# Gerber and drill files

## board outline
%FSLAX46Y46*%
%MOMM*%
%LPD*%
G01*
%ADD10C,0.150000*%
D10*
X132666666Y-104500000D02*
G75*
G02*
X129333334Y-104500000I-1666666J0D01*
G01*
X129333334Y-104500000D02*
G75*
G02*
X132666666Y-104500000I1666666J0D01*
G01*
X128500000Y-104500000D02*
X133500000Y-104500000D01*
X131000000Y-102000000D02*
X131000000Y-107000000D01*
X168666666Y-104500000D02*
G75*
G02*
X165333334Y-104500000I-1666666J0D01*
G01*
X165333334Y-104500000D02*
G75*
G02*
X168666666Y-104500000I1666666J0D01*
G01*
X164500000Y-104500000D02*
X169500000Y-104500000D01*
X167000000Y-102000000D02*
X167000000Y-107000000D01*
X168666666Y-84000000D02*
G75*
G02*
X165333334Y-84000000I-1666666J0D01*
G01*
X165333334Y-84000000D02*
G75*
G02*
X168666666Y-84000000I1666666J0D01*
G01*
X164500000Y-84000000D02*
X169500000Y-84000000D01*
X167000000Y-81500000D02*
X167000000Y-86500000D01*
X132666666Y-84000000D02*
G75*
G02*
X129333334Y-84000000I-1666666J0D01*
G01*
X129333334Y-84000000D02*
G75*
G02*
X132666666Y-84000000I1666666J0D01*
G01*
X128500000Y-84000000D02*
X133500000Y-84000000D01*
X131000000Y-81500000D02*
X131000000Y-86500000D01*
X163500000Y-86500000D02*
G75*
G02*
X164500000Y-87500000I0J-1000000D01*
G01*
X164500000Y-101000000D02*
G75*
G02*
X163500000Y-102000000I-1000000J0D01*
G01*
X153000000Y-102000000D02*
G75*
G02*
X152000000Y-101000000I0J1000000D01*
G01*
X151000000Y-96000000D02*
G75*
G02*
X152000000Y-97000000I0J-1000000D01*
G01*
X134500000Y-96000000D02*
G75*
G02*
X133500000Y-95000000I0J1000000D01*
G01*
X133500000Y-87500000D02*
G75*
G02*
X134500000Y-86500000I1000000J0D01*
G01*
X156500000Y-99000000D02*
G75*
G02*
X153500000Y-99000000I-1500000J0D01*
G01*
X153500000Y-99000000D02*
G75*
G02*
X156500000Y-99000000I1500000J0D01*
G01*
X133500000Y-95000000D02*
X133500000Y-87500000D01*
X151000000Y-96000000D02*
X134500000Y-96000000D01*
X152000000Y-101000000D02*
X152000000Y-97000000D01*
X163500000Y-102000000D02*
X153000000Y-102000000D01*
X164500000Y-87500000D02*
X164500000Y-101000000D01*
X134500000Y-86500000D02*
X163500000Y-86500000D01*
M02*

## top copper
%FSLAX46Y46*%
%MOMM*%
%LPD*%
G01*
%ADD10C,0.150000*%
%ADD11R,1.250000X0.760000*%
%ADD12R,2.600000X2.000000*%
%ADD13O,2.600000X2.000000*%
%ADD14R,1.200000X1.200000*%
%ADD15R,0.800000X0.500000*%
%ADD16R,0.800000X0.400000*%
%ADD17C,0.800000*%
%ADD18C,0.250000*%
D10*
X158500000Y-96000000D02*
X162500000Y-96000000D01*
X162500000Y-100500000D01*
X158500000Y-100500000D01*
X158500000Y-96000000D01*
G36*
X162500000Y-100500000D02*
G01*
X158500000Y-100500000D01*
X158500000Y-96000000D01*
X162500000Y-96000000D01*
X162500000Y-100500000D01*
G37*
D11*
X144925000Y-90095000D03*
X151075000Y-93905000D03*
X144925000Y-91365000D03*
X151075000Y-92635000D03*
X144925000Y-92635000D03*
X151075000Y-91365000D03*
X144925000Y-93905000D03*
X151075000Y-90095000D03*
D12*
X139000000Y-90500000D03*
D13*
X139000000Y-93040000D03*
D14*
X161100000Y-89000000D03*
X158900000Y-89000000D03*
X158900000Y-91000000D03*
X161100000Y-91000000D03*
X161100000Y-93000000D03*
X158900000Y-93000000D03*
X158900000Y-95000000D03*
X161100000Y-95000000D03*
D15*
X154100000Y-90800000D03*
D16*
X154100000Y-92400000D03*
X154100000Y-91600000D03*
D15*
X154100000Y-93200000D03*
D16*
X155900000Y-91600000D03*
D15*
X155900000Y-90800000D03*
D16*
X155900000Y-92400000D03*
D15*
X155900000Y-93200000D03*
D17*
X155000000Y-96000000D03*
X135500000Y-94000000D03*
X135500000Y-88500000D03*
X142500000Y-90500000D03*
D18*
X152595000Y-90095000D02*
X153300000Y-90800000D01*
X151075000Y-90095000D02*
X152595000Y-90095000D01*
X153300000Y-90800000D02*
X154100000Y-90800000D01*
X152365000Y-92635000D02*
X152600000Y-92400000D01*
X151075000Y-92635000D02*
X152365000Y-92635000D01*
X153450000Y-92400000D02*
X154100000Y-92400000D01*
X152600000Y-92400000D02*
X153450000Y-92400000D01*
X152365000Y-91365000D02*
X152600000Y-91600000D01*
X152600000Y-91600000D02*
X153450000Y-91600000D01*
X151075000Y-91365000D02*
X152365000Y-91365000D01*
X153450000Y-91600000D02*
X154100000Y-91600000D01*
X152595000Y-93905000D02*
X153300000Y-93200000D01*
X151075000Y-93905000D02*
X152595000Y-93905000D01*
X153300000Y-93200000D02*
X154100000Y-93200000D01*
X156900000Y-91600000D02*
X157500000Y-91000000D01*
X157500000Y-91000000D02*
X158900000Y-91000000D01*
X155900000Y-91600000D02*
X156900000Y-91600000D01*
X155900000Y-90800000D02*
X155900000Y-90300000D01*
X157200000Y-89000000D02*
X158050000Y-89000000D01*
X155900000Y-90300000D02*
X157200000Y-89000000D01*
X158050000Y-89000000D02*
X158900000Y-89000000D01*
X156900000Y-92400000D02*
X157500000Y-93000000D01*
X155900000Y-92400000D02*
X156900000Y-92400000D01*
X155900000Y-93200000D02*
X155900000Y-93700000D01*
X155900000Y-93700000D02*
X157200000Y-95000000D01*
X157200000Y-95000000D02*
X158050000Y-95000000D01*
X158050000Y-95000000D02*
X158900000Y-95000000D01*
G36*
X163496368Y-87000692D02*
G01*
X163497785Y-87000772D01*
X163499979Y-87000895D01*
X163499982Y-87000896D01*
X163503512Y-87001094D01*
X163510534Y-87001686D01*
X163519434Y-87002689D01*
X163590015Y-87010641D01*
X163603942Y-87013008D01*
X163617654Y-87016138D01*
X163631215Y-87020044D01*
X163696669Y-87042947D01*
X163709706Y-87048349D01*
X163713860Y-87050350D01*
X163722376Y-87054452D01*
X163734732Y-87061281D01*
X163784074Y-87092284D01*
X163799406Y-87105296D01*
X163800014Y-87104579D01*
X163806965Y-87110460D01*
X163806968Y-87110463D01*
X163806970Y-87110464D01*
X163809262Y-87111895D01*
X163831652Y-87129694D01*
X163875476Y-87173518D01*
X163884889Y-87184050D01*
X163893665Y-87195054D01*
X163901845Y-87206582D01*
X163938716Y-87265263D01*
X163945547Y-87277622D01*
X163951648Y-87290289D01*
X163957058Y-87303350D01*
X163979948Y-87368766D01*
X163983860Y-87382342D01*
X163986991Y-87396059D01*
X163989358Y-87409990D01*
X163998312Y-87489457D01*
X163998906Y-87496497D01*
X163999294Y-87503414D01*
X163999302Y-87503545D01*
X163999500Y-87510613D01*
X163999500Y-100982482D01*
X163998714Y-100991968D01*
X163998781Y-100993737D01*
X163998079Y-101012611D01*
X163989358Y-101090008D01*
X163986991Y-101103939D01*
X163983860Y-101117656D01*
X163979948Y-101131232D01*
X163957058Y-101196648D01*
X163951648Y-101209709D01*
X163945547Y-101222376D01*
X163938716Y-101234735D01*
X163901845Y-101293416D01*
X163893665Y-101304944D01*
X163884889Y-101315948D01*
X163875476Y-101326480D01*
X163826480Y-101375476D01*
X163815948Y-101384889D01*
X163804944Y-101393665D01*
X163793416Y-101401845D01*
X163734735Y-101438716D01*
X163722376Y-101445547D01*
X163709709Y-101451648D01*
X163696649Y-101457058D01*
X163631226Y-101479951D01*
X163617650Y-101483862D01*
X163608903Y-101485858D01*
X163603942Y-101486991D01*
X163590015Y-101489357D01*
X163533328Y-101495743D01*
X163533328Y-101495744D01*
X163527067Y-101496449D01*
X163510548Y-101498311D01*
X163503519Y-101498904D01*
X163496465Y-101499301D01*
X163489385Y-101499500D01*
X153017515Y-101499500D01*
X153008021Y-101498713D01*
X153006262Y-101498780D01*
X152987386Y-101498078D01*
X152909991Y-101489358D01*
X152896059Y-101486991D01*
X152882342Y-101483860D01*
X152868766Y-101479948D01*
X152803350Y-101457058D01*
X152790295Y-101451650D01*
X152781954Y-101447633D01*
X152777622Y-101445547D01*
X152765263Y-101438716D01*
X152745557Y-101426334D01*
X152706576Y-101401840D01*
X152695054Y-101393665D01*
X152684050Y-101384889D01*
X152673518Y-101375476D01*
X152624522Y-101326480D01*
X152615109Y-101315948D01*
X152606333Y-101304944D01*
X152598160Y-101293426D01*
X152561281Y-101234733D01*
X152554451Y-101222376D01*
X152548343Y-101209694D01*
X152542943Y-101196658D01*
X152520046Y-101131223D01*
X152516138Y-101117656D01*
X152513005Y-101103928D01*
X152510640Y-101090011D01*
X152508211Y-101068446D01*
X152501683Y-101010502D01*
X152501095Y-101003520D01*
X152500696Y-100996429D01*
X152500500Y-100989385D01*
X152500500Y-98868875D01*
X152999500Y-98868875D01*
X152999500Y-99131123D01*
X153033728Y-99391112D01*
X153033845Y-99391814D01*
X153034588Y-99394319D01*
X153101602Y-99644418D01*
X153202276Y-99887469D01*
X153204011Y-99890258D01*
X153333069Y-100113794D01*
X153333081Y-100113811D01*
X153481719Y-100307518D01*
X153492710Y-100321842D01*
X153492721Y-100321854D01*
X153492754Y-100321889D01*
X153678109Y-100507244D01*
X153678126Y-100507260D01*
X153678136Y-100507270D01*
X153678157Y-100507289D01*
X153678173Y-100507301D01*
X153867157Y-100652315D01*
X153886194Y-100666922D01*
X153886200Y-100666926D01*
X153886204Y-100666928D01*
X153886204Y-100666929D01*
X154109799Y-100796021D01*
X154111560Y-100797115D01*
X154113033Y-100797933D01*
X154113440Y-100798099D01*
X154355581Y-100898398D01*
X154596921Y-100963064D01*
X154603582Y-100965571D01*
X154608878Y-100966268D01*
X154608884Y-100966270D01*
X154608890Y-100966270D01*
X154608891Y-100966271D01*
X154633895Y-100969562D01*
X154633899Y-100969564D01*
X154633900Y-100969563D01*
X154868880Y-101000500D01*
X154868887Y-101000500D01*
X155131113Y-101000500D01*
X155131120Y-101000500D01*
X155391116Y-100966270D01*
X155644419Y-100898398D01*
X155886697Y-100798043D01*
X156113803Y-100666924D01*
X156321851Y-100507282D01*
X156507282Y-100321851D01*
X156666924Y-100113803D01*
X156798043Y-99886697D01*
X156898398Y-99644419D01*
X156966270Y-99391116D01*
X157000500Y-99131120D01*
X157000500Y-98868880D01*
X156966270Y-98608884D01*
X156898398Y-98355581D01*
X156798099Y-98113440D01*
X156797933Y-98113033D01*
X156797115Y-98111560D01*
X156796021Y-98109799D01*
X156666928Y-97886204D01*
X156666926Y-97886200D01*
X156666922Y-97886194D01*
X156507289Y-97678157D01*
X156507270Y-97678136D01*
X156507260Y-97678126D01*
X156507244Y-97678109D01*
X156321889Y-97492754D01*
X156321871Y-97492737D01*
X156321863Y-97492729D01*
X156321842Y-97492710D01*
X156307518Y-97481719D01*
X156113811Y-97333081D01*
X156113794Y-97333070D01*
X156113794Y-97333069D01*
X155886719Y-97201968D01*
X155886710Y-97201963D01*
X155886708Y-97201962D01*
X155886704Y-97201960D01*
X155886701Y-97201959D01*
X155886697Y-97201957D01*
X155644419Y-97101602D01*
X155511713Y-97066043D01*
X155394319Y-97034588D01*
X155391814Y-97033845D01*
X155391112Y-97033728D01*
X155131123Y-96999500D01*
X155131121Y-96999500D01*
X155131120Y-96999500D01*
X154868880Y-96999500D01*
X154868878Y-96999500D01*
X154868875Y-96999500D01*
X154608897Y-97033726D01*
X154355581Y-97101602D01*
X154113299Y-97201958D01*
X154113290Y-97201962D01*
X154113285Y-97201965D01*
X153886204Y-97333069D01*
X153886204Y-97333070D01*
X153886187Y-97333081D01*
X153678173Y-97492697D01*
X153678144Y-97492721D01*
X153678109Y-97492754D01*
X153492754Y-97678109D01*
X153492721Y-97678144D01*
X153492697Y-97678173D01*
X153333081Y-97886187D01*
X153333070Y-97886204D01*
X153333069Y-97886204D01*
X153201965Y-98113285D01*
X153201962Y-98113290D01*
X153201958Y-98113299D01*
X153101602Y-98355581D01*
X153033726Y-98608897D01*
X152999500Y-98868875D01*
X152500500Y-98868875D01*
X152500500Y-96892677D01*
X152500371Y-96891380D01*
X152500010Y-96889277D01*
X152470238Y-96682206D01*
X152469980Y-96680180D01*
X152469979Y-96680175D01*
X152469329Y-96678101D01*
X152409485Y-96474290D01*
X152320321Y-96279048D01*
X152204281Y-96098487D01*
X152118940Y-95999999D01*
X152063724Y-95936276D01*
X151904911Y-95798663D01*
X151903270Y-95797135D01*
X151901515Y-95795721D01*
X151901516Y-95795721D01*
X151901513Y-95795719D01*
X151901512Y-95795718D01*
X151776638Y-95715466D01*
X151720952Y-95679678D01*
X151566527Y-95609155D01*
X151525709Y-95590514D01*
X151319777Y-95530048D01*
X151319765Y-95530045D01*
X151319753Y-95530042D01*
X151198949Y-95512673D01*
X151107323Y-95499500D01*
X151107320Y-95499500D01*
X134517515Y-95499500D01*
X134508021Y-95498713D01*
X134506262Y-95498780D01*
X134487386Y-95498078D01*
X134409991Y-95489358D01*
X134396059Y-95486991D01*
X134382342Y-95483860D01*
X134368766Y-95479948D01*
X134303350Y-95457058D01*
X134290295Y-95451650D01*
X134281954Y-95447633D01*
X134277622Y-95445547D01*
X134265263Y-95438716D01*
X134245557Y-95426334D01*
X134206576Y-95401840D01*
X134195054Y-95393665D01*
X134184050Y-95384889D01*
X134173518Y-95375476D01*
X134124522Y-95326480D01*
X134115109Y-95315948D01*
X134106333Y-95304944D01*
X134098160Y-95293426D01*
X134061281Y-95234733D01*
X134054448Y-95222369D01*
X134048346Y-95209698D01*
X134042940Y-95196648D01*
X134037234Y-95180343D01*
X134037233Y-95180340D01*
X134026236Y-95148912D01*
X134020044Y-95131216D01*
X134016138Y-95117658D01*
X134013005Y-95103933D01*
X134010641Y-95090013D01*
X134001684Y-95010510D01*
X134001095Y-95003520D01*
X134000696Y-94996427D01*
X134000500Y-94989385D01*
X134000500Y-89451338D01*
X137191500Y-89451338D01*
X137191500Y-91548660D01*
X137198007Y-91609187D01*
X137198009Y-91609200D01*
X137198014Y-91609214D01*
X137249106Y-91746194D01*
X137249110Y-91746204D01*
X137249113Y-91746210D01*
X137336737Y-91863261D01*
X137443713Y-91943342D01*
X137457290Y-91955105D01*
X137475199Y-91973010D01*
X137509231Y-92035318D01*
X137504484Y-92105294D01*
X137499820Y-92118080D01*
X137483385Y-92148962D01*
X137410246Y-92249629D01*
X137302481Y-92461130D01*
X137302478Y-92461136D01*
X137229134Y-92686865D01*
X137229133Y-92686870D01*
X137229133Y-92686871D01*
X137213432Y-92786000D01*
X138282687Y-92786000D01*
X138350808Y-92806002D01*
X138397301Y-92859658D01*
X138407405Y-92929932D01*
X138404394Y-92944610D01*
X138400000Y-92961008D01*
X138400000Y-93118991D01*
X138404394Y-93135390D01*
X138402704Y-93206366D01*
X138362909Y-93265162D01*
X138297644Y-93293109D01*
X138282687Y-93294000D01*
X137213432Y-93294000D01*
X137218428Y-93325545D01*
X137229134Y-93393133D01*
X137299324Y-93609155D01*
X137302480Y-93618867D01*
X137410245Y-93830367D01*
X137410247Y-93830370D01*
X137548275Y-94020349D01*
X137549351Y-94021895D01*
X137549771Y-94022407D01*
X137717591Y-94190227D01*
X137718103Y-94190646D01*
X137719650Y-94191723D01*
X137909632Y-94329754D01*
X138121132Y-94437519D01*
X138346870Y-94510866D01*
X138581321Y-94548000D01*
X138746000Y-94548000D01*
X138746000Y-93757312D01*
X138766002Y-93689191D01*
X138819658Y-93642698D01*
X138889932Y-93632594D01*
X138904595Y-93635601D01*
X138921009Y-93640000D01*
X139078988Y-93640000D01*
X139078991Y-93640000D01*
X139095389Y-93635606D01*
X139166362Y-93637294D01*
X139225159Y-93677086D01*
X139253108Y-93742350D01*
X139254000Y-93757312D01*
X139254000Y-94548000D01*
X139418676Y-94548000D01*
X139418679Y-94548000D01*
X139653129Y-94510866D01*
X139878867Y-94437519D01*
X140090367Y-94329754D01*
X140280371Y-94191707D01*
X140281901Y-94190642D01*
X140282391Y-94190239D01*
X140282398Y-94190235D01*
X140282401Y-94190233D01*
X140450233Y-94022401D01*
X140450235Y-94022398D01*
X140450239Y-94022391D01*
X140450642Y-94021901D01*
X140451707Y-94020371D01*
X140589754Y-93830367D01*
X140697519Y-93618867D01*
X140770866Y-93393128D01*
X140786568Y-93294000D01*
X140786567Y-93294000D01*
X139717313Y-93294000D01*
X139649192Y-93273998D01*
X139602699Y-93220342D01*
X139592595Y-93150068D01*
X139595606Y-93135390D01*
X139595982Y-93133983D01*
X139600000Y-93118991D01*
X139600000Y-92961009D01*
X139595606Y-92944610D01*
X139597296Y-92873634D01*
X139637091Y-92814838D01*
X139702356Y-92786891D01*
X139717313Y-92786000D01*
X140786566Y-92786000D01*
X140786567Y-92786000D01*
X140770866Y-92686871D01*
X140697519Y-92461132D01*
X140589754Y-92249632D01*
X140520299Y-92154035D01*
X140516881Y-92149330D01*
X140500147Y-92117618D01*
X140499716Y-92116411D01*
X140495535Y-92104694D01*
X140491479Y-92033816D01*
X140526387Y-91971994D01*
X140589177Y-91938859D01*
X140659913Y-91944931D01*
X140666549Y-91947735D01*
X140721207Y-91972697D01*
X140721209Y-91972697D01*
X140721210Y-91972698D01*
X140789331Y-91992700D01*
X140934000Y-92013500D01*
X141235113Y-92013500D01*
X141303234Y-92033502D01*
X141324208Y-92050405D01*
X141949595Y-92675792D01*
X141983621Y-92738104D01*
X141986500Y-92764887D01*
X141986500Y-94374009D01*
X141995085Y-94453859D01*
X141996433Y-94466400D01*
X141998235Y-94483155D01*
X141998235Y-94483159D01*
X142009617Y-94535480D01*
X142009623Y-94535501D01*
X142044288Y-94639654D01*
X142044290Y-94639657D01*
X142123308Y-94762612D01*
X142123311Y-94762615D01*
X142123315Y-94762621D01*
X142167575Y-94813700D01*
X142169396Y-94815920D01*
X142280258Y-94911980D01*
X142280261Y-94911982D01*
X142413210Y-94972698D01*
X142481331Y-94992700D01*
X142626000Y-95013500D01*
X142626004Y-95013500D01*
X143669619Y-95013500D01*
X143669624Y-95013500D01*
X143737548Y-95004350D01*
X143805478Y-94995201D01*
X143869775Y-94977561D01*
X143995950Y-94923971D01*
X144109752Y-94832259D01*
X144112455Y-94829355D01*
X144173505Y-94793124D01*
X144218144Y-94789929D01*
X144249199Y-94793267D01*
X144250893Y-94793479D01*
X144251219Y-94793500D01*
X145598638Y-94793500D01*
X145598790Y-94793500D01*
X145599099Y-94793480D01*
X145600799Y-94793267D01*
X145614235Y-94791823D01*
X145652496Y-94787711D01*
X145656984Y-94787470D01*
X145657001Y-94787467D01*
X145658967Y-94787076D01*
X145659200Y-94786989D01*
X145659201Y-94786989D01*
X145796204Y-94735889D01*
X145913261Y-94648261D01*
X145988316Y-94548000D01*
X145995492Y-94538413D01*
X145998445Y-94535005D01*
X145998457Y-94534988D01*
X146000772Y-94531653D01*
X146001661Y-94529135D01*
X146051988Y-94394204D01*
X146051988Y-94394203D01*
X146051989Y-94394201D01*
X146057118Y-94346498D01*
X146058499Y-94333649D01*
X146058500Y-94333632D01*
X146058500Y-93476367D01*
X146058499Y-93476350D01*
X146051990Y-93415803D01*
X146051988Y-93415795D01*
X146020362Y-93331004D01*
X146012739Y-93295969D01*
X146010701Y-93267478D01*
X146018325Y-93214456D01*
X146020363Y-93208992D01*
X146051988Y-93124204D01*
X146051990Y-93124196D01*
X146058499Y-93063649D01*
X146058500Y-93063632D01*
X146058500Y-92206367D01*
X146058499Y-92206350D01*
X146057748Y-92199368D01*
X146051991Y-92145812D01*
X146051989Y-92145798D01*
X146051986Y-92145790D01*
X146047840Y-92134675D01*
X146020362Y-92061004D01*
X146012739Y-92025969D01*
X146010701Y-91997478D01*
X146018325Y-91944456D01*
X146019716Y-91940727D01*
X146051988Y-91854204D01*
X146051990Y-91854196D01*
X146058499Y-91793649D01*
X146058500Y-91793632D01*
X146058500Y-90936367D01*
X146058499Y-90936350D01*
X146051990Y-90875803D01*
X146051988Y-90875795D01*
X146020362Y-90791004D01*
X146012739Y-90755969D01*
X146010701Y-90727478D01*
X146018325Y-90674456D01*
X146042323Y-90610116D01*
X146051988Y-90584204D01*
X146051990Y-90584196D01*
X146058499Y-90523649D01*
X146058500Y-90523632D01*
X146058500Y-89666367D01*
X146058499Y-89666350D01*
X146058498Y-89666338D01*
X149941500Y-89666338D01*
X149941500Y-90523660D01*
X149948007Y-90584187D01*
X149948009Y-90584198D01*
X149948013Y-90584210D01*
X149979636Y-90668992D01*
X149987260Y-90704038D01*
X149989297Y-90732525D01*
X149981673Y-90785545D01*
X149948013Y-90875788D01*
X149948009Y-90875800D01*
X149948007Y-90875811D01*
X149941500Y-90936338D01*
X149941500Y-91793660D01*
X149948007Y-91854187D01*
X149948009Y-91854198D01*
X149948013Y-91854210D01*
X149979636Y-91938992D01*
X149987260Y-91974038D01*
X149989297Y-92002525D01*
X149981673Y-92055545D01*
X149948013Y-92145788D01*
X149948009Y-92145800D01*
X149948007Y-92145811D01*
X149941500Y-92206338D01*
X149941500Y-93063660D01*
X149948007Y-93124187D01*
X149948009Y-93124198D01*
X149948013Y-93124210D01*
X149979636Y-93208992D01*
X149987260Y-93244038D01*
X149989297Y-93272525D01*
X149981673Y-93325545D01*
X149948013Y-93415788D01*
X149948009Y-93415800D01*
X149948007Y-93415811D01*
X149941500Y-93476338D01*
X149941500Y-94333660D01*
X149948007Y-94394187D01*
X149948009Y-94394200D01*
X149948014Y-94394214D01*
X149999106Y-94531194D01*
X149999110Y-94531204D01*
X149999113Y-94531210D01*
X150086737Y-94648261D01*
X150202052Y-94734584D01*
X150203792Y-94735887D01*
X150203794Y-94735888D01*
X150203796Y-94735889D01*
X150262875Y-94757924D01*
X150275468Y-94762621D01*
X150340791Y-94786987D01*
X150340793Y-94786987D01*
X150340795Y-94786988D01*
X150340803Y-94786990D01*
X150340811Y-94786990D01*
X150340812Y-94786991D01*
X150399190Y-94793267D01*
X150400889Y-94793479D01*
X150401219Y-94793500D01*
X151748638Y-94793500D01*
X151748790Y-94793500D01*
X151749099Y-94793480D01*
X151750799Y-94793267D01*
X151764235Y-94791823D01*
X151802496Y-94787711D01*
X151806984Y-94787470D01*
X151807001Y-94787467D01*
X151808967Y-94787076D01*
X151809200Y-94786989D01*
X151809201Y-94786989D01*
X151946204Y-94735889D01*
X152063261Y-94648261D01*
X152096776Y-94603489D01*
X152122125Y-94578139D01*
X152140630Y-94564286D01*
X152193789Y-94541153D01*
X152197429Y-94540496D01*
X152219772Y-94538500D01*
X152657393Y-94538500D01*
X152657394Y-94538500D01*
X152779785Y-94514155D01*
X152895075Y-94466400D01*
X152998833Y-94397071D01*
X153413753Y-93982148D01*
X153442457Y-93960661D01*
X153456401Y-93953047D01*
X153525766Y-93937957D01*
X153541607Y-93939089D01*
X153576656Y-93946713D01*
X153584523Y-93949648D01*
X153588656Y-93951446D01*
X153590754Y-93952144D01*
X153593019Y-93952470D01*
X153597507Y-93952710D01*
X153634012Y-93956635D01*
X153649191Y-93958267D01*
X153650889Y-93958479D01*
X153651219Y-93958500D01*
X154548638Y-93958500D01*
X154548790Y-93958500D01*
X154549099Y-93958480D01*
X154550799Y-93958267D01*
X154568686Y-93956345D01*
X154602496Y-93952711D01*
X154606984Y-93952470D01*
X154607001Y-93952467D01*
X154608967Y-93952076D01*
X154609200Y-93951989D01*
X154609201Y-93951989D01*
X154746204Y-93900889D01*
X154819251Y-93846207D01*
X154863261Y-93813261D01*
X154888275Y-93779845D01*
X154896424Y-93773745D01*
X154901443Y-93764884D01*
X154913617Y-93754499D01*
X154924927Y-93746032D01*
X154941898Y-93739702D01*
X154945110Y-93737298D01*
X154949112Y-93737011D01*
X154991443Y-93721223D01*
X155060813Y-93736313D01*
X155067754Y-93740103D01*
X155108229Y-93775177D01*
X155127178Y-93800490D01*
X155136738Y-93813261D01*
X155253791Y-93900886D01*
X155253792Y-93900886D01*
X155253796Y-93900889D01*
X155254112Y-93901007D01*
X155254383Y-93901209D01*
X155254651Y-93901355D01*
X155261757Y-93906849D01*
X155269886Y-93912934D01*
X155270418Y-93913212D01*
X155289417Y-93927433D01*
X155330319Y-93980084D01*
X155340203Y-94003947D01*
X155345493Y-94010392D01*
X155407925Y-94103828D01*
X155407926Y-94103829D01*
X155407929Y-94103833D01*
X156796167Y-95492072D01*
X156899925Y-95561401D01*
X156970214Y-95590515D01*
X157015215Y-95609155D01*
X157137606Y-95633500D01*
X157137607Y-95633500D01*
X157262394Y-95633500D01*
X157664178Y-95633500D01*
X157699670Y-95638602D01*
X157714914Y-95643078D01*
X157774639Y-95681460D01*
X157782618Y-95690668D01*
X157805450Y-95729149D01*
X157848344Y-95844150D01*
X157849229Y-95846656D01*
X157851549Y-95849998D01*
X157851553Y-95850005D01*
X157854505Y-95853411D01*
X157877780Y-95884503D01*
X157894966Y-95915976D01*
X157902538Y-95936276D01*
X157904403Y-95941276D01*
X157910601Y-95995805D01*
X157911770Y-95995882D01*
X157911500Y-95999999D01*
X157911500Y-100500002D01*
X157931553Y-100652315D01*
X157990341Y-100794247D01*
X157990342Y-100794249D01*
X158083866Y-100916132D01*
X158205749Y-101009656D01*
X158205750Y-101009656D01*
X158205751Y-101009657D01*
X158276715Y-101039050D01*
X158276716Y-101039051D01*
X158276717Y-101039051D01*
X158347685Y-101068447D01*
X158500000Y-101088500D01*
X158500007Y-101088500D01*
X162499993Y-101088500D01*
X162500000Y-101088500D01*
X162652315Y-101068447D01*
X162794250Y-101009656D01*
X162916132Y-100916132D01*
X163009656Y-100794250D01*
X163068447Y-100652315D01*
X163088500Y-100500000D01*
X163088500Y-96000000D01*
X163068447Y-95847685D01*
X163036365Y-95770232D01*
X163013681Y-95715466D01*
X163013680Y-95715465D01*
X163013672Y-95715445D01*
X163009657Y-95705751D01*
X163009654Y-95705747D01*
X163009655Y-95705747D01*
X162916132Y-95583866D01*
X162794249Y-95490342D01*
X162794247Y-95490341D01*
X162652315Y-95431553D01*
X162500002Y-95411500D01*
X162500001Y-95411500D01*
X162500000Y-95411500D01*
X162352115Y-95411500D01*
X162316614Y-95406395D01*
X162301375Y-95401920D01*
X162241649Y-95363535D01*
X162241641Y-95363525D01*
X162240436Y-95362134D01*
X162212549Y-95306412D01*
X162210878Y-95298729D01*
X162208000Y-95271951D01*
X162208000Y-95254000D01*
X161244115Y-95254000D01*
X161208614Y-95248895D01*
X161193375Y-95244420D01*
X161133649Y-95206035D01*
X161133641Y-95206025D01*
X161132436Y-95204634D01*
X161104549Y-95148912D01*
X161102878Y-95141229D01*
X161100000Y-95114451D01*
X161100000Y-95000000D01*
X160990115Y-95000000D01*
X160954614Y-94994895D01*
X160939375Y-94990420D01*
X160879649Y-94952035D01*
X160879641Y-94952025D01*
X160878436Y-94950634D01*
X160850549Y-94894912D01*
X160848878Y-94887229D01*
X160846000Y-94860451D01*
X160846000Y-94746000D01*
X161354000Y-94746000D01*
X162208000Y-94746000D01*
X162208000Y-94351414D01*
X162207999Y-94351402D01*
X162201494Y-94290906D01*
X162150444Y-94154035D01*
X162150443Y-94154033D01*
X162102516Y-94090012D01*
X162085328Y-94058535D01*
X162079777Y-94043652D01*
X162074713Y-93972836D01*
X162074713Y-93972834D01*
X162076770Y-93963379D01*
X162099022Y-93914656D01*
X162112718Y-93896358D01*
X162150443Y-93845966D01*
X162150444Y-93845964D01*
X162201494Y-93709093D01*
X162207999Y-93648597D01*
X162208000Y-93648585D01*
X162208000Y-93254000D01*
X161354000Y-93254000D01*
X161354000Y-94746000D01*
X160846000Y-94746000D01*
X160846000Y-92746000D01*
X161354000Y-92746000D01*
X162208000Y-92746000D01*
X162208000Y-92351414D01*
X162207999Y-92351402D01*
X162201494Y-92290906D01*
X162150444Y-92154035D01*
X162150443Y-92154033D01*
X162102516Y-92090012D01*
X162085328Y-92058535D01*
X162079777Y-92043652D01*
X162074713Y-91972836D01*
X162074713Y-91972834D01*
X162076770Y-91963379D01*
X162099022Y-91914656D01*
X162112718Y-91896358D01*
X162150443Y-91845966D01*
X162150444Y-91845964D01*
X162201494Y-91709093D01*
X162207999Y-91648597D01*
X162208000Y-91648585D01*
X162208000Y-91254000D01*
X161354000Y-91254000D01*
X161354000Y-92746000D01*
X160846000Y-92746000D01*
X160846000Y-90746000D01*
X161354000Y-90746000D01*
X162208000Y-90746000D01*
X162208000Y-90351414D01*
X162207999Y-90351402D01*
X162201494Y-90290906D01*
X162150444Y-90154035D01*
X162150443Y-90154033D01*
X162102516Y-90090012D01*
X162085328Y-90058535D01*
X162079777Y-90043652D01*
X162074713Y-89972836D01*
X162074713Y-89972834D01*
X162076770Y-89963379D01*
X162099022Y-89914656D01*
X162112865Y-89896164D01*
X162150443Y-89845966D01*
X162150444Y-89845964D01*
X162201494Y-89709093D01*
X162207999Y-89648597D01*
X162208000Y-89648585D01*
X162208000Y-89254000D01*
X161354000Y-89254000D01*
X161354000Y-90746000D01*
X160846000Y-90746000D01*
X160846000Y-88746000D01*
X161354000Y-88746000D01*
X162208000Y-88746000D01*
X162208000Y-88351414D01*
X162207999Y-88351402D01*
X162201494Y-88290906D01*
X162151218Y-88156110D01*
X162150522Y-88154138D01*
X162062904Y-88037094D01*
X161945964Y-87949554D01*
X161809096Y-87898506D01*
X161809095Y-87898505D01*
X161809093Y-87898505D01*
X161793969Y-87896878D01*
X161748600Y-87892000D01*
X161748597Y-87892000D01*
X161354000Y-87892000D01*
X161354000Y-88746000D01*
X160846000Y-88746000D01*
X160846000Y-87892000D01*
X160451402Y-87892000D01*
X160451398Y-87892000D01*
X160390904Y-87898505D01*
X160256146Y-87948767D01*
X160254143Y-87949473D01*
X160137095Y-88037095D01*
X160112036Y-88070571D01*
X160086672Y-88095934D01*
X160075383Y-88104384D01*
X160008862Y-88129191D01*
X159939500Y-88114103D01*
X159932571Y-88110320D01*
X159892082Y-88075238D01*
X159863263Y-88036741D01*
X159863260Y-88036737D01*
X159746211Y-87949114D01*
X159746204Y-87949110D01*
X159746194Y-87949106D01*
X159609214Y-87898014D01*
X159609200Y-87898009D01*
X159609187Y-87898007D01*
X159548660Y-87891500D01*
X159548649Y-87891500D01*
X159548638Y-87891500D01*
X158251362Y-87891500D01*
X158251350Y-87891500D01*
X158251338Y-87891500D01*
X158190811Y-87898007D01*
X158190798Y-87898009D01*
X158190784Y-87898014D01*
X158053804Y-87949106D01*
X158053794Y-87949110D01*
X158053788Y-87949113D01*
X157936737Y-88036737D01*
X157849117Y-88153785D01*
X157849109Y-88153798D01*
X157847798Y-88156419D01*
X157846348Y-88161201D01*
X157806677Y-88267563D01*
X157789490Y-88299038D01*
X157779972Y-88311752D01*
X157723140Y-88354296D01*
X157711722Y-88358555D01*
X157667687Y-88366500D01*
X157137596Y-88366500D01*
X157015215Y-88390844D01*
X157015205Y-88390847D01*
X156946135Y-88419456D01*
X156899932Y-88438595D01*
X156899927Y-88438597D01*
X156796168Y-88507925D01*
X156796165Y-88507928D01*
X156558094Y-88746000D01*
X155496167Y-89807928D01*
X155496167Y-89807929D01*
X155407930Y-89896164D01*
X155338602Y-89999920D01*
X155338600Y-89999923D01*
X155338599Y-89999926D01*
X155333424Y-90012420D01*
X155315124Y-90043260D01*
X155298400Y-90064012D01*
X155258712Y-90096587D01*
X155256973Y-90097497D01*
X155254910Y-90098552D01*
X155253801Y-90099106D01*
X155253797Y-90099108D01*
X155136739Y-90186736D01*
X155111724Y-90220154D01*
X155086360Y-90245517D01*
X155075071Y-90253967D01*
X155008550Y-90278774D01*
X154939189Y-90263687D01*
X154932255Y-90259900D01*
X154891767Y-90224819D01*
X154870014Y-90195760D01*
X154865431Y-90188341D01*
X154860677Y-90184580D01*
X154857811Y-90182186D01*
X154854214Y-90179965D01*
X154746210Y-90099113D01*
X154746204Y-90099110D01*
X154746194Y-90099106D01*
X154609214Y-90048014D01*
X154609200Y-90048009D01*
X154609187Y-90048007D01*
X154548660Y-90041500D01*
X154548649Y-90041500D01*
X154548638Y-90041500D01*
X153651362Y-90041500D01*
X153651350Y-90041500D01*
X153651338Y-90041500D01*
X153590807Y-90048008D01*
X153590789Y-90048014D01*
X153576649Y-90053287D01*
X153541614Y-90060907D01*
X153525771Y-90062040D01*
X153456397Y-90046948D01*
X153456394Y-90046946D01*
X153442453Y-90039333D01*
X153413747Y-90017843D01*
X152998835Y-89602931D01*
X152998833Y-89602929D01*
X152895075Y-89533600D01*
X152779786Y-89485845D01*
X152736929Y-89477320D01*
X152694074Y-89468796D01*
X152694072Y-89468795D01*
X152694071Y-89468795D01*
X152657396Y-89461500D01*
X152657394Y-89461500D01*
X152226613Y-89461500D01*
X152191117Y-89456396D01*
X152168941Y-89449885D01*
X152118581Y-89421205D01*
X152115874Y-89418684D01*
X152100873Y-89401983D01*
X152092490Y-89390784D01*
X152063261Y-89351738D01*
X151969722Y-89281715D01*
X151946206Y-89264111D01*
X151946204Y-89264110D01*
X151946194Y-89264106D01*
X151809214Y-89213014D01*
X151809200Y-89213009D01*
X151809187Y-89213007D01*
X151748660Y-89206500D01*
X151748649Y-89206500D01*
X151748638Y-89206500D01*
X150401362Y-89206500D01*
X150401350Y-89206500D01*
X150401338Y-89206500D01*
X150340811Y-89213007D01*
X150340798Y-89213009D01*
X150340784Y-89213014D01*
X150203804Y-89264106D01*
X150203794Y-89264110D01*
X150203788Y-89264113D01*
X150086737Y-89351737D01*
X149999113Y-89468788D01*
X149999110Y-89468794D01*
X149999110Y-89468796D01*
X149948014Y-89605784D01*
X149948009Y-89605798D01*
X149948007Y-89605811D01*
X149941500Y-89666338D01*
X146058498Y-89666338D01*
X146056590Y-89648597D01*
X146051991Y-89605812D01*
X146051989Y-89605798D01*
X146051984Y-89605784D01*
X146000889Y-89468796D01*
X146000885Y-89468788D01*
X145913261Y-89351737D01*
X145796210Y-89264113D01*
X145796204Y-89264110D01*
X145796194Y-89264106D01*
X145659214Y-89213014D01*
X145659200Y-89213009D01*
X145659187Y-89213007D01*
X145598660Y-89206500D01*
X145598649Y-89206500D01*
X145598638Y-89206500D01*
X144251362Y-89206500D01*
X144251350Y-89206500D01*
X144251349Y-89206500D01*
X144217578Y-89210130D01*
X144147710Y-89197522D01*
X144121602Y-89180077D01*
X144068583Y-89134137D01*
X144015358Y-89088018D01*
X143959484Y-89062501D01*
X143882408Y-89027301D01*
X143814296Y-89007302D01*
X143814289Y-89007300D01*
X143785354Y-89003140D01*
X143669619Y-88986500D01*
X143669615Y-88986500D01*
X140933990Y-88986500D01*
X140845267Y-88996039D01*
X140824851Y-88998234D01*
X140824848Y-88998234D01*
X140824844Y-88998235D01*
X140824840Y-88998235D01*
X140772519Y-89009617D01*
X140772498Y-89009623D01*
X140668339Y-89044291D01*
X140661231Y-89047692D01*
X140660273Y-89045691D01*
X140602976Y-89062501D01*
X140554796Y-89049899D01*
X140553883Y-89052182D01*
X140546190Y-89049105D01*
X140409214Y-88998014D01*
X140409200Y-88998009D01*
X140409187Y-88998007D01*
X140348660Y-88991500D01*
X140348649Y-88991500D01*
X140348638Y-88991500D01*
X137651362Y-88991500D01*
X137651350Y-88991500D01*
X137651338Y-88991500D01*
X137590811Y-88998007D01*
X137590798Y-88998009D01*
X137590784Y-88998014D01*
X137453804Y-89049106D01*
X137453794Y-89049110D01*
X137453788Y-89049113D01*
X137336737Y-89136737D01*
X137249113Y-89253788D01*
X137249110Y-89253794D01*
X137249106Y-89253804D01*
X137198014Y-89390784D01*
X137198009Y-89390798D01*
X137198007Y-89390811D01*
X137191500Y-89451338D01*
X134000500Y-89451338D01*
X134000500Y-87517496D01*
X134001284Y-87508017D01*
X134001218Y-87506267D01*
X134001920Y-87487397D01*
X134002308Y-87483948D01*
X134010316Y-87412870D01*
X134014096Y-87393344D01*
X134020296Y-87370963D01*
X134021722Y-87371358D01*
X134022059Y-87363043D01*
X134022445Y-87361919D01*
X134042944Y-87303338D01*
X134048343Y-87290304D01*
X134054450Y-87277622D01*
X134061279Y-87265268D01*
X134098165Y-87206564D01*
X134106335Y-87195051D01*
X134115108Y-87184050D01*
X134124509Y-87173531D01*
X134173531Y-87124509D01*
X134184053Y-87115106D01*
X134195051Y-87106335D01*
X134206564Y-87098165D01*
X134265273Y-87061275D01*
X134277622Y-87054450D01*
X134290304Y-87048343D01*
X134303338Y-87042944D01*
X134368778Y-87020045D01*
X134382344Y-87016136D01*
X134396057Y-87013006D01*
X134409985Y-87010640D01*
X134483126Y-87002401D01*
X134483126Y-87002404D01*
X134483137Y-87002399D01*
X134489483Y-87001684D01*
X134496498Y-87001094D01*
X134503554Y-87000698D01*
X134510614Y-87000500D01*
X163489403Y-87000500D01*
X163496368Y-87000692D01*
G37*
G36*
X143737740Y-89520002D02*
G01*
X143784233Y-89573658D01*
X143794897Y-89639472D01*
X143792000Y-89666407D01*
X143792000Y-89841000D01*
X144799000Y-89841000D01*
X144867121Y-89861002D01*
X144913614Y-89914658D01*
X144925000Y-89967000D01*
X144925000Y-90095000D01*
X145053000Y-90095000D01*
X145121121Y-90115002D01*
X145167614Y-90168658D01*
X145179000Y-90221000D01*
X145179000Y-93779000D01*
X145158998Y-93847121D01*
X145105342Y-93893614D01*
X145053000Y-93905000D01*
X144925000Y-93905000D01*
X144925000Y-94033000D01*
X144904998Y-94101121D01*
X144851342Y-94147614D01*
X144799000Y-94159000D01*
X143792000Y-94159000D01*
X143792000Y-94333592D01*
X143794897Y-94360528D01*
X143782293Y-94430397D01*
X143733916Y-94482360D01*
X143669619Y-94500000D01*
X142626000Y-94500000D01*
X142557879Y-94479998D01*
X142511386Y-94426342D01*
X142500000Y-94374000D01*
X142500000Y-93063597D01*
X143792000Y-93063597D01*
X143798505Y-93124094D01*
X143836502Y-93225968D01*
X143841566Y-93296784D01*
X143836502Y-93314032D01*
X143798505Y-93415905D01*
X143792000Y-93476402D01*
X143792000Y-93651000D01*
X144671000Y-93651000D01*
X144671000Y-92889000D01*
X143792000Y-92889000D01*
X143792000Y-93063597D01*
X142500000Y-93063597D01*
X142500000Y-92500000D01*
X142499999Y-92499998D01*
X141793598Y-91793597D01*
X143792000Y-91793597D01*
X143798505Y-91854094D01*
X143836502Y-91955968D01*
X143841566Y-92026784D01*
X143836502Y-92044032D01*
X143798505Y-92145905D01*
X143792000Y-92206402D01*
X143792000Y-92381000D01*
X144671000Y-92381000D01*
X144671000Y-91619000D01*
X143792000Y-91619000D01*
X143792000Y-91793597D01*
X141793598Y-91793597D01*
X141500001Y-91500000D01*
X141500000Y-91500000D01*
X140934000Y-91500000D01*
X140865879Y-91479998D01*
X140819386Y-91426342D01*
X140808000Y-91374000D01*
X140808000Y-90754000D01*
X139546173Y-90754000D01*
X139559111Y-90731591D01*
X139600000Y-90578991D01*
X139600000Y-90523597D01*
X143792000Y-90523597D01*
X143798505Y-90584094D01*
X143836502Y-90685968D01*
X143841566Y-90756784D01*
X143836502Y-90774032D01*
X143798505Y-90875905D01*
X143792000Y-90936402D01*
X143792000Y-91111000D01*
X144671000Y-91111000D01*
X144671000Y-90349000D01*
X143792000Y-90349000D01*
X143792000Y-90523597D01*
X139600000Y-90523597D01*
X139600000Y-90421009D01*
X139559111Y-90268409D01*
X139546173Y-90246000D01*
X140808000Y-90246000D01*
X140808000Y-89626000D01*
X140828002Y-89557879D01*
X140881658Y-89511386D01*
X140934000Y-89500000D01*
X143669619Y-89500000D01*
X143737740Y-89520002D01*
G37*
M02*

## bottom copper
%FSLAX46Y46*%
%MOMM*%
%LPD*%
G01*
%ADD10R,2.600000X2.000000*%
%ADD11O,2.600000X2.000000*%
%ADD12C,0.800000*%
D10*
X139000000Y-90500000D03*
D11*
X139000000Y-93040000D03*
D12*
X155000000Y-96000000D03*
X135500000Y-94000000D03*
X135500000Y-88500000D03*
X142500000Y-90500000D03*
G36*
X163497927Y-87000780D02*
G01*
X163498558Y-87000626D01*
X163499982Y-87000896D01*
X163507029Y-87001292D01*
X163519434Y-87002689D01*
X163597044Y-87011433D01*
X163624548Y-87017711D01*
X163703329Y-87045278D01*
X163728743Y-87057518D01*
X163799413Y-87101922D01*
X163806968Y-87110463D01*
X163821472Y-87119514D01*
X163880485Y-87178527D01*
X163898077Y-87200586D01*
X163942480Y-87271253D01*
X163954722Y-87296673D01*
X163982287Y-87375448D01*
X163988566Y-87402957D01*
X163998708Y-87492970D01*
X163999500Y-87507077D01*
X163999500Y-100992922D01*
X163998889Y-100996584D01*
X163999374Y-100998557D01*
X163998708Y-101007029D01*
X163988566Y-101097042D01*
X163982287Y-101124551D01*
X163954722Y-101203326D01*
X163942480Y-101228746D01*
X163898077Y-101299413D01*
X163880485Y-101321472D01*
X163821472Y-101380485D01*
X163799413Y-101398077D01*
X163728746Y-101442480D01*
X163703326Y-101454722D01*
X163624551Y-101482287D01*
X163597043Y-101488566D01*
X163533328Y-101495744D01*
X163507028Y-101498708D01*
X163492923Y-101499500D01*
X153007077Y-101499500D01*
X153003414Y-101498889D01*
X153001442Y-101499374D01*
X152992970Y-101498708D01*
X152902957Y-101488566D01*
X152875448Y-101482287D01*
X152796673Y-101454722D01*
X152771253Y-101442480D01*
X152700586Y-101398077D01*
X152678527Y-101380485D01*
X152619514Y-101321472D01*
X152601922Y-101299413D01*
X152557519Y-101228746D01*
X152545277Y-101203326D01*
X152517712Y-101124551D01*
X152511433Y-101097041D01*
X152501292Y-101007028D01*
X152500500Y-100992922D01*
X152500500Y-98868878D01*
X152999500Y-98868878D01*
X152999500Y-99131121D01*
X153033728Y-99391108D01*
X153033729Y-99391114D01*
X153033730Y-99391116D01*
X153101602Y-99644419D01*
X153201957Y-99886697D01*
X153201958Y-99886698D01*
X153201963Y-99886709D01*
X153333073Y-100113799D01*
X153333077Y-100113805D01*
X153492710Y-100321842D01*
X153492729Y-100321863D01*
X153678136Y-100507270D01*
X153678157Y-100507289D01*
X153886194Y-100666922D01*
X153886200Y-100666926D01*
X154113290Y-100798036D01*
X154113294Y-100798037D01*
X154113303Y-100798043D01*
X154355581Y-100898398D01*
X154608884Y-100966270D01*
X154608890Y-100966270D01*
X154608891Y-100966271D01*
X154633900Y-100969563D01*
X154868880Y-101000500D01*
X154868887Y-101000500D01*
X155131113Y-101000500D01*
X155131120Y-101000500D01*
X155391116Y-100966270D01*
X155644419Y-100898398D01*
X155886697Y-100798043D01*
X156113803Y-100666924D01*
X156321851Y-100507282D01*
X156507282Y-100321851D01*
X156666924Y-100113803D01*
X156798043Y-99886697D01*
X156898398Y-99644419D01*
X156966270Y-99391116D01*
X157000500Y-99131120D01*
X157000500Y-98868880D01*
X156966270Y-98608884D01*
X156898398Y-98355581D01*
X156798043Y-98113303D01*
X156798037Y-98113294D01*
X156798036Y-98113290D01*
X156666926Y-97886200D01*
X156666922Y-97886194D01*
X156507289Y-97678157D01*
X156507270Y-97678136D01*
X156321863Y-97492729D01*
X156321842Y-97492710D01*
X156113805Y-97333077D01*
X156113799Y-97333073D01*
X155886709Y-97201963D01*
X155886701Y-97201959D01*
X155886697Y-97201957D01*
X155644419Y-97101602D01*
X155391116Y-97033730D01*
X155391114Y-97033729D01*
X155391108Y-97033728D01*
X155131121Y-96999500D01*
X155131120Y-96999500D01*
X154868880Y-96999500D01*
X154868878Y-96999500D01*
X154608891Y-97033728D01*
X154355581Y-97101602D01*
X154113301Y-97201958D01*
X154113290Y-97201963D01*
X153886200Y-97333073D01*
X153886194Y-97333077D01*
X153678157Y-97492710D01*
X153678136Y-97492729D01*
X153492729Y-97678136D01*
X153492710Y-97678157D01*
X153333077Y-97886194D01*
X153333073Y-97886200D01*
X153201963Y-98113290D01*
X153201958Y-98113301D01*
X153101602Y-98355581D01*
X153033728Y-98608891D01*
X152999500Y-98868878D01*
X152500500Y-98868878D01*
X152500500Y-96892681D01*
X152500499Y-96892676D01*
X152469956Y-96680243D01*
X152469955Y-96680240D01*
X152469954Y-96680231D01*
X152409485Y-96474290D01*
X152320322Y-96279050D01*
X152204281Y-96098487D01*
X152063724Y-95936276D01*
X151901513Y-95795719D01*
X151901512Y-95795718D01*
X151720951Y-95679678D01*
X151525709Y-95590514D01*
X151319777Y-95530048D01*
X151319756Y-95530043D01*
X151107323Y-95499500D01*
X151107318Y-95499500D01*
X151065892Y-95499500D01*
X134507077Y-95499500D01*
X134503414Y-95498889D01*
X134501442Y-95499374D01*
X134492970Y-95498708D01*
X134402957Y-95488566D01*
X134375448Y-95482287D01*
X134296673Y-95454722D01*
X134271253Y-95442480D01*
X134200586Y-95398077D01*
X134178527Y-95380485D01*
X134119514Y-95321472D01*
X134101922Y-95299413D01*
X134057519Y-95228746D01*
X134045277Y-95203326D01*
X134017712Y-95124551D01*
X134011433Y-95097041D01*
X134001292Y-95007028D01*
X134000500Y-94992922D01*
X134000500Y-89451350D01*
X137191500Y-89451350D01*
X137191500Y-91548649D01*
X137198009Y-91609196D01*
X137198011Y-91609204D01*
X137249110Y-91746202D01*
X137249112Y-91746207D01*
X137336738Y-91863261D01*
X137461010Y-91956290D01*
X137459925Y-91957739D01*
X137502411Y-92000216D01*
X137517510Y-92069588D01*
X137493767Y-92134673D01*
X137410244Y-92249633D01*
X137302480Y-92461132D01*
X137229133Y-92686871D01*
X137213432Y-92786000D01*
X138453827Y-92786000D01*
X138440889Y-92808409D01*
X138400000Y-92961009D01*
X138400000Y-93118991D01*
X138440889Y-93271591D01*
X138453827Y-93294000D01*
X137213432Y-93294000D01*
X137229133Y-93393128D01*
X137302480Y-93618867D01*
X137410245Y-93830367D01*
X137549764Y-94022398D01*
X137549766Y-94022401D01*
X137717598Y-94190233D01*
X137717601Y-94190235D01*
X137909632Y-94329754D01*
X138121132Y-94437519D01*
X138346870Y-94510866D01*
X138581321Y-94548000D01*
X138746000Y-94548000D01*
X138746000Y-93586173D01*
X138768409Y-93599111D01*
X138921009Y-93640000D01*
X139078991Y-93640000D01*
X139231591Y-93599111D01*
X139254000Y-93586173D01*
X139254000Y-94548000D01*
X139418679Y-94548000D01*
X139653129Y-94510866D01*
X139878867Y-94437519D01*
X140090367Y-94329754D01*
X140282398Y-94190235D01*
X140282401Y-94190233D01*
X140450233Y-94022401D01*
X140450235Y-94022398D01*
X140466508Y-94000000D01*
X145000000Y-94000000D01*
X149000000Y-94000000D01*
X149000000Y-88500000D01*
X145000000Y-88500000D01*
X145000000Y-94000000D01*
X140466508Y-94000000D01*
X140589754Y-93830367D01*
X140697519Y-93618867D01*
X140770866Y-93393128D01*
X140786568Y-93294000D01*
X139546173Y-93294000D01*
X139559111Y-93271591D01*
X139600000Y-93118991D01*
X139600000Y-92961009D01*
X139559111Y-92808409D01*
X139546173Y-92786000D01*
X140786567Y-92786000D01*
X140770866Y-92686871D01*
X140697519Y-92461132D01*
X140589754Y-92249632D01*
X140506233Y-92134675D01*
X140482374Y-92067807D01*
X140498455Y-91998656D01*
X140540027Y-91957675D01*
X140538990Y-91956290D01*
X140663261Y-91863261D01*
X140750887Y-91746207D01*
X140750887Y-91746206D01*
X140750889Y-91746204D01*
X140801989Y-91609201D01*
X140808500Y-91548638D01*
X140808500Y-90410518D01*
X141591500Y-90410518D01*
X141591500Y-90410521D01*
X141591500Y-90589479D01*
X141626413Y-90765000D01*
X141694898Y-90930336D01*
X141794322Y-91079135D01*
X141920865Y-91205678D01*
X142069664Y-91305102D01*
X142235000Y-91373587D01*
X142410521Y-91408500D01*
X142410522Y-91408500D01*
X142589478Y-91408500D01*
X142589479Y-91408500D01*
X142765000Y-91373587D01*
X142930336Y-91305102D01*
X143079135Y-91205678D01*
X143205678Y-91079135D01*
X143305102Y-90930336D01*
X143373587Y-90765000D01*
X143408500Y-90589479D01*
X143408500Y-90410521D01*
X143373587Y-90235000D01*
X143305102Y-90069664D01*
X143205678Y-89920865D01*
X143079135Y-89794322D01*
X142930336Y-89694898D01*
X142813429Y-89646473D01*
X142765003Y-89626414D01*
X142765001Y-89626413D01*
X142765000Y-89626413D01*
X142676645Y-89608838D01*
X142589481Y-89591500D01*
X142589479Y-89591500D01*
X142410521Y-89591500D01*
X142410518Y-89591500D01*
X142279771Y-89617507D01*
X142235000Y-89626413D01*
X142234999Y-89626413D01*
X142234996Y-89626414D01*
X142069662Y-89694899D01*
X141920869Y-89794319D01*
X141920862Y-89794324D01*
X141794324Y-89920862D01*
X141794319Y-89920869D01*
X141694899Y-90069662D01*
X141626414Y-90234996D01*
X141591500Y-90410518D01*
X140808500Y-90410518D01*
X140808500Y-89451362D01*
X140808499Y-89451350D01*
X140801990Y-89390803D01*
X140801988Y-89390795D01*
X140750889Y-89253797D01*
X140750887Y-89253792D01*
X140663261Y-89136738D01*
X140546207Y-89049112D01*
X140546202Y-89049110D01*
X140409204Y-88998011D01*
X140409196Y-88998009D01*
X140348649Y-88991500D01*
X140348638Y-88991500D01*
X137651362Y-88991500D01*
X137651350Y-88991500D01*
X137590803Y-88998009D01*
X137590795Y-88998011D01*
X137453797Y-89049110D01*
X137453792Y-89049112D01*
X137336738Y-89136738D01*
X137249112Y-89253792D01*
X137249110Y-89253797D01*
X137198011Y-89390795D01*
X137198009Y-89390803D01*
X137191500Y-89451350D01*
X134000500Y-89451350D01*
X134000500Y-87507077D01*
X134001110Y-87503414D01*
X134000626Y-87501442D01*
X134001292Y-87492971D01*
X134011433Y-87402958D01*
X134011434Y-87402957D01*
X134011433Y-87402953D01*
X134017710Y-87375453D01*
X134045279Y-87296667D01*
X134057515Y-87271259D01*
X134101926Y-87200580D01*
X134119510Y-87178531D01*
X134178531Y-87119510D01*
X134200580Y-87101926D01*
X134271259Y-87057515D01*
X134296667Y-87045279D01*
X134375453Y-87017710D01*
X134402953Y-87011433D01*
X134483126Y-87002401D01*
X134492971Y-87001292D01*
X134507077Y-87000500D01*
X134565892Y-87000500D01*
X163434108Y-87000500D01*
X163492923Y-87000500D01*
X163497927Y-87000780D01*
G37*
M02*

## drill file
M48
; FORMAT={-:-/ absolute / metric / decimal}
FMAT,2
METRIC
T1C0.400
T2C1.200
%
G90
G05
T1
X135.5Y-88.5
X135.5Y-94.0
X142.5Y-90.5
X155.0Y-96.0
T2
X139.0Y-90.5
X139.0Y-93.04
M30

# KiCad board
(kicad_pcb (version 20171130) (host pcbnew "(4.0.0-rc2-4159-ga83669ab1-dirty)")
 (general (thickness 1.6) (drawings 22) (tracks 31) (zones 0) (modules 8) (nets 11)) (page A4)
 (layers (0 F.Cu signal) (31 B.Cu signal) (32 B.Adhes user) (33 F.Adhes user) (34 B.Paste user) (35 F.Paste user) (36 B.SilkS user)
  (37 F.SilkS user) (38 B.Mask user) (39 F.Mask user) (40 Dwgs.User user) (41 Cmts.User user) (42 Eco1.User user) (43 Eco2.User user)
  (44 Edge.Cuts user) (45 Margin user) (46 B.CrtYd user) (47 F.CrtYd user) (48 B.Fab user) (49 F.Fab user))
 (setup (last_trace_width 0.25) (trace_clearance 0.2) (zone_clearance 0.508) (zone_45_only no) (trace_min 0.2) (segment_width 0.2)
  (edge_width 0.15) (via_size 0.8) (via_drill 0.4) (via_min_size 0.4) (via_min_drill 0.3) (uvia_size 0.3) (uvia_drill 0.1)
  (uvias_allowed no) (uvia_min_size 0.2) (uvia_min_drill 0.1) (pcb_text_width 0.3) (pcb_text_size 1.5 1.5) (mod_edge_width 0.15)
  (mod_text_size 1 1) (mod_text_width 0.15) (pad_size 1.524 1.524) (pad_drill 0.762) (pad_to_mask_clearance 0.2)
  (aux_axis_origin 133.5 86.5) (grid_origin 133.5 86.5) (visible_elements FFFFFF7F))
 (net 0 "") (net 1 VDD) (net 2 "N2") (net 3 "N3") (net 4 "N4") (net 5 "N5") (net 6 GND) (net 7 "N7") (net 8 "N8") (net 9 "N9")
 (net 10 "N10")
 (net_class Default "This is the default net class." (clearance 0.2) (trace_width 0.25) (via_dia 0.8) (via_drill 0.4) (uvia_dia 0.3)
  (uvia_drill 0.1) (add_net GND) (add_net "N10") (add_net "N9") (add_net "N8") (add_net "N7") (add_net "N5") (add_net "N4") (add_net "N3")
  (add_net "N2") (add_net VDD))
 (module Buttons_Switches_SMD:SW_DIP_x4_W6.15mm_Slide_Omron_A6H (layer F.Cu) (at 148 92)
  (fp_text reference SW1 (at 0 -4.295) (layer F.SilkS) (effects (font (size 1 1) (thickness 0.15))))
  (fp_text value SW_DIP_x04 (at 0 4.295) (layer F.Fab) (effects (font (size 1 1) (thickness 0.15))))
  (pad 1 smd rect (at -3.075 -1.905) (size 1.25 0.76) (layers F.Cu F.Mask) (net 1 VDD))
  (pad 5 smd rect (at 3.075 1.905) (size 1.25 0.76) (layers F.Cu F.Mask) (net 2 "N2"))
  (pad 2 smd rect (at -3.075 -0.635) (size 1.25 0.76) (layers F.Cu F.Mask) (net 1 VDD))
  (pad 6 smd rect (at 3.075 0.635) (size 1.25 0.76) (layers F.Cu F.Mask) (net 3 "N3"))
  (pad 3 smd rect (at -3.075 0.635) (size 1.25 0.76) (layers F.Cu F.Mask) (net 1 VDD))
  (pad 7 smd rect (at 3.075 -0.635) (size 1.25 0.76) (layers F.Cu F.Mask) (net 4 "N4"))
  (pad 4 smd rect (at -3.075 1.905) (size 1.25 0.76) (layers F.Cu F.Mask) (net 1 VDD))
  (pad 8 smd rect (at 3.075 -1.905) (size 1.25 0.76) (layers F.Cu F.Mask) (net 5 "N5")))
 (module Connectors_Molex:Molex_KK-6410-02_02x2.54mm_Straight (layer F.Cu) (at 139 90.5 270)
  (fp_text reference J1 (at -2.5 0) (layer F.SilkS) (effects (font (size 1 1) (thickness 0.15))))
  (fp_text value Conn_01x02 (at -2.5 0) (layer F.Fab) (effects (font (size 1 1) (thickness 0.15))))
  (pad 1 thru_hole rect (at 0 0 270) (size 2 2.6) (drill 1.2) (layers *.Cu *.Mask) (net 1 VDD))
  (pad 2 thru_hole oval (at 2.54 0 270) (size 2 2.6) (drill 1.2) (layers *.Cu *.Mask) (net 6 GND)))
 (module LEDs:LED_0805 (layer F.Cu) (at 160 89 180)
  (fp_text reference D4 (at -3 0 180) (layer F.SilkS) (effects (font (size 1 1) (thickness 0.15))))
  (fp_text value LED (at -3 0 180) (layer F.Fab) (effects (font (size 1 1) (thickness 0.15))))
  (pad 1 smd rect (at -1.1 0) (size 1.2 1.2) (layers F.Cu F.Paste F.Mask) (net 6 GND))
  (pad 2 smd rect (at 1.1 0) (size 1.2 1.2) (layers F.Cu F.Paste F.Mask) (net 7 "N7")))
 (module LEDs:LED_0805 (layer F.Cu) (at 160 91 180)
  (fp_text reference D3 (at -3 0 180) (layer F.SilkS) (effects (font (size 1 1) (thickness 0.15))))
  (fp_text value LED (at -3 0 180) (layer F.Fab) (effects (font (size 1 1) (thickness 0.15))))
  (pad 2 smd rect (at 1.1 0) (size 1.2 1.2) (layers F.Cu F.Paste F.Mask) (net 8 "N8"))
  (pad 1 smd rect (at -1.1 0) (size 1.2 1.2) (layers F.Cu F.Paste F.Mask) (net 6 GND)))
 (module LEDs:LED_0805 (layer F.Cu) (at 160 93 180)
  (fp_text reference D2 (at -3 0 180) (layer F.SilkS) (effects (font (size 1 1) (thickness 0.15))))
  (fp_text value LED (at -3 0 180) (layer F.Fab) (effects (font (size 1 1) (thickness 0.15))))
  (pad 1 smd rect (at -1.1 0) (size 1.2 1.2) (layers F.Cu F.Paste F.Mask) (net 6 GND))
  (pad 2 smd rect (at 1.1 0) (size 1.2 1.2) (layers F.Cu F.Paste F.Mask) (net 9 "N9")))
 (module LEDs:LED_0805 (layer F.Cu) (at 160 95 180)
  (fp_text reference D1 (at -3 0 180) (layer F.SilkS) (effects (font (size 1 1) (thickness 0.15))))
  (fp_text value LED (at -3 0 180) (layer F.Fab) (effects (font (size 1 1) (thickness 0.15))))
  (pad 2 smd rect (at 1.1 0) (size 1.2 1.2) (layers F.Cu F.Paste F.Mask) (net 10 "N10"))
  (pad 1 smd rect (at -1.1 0) (size 1.2 1.2) (layers F.Cu F.Paste F.Mask) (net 6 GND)))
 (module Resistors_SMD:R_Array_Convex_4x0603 (layer F.Cu) (at 155 92)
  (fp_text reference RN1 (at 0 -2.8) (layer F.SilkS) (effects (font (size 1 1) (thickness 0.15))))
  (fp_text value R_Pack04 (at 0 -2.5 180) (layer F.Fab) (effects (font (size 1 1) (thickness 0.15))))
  (pad 1 smd rect (at -0.9 -1.2) (size 0.8 0.5) (layers F.Cu F.Paste F.Mask) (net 5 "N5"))
  (pad 3 smd rect (at -0.9 0.4) (size 0.8 0.4) (layers F.Cu F.Paste F.Mask) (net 3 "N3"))
  (pad 2 smd rect (at -0.9 -0.4) (size 0.8 0.4) (layers F.Cu F.Paste F.Mask) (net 4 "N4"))
  (pad 4 smd rect (at -0.9 1.2) (size 0.8 0.5) (layers F.Cu F.Paste F.Mask) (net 2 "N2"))
  (pad 7 smd rect (at 0.9 -0.4) (size 0.8 0.4) (layers F.Cu F.Paste F.Mask) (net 8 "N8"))
  (pad 8 smd rect (at 0.9 -1.2) (size 0.8 0.5) (layers F.Cu F.Paste F.Mask) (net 7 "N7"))
  (pad 6 smd rect (at 0.9 0.4) (size 0.8 0.4) (layers F.Cu F.Paste F.Mask) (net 9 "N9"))
  (pad 5 smd rect (at 0.9 1.2) (size 0.8 0.5) (layers F.Cu F.Paste F.Mask) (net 10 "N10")))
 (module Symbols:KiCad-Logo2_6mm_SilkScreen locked (layer B.Cu) (at 156.5 91 180)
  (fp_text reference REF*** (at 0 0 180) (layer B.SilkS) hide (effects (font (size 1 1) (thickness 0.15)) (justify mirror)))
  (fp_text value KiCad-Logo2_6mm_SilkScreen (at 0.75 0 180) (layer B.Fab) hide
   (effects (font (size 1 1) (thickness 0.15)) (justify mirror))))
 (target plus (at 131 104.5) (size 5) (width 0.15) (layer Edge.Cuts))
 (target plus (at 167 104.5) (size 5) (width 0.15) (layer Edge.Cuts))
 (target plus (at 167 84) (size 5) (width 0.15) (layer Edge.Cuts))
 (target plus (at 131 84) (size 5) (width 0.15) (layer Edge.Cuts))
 (gr_poly (pts (xy 158.5 96) (xy 162.5 96) (xy 162.5 100.5) (xy 158.5 100.5)) (layer F.Cu) (width 0.15))
 (gr_arc (start 163.5 87.5) (end 164.5 87.5) (angle -90) (layer Edge.Cuts) (width 0.15))
 (gr_arc (start 163.5 101) (end 163.5 102) (angle -90) (layer Edge.Cuts) (width 0.15))
 (gr_arc (start 153 101) (end 152 101) (angle -90) (layer Edge.Cuts) (width 0.15))
 (gr_arc (start 151 97) (end 152 97) (angle -90) (layer Edge.Cuts) (width 0.15))
 (gr_arc (start 134.5 95) (end 133.5 95) (angle -90) (layer Edge.Cuts) (width 0.15))
 (gr_arc (start 134.5 87.5) (end 134.5 86.5) (angle -90) (layer Edge.Cuts) (width 0.15))
 (gr_circle (center 155 99) (end 156.5 99) (layer Edge.Cuts) (width 0.15))
 (gr_line (start 133.5 95) (end 133.5 87.5) (layer Edge.Cuts) (width 0.15))
 (gr_line (start 151 96) (end 134.5 96) (layer Edge.Cuts) (width 0.15))
 (gr_line (start 152 101) (end 152 97) (layer Edge.Cuts) (width 0.15))
 (gr_line (start 163.5 102) (end 153 102) (layer Edge.Cuts) (width 0.15))
 (gr_line (start 164.5 87.5) (end 164.5 101) (layer Edge.Cuts) (width 0.15))
 (gr_line (start 134.5 86.5) (end 163.5 86.5) (layer Edge.Cuts) (width 0.15))
 (segment (start 152.595 90.095) (end 153.3 90.8) (width 0.25) (layer F.Cu) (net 5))
 (segment (start 151.075 90.095) (end 152.595 90.095) (width 0.25) (layer F.Cu) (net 5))
 (segment (start 153.3 90.8) (end 154.1 90.8) (width 0.25) (layer F.Cu) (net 5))
 (segment (start 152.365 92.635) (end 152.6 92.4) (width 0.25) (layer F.Cu) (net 3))
 (segment (start 151.075 92.635) (end 152.365 92.635) (width 0.25) (layer F.Cu) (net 3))
 (segment (start 153.45 92.4) (end 154.1 92.4) (width 0.25) (layer F.Cu) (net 3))
 (segment (start 152.6 92.4) (end 153.45 92.4) (width 0.25) (layer F.Cu) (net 3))
 (segment (start 152.365 91.365) (end 152.6 91.6) (width 0.25) (layer F.Cu) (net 4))
 (segment (start 152.6 91.6) (end 153.45 91.6) (width 0.25) (layer F.Cu) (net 4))
 (segment (start 151.075 91.365) (end 152.365 91.365) (width 0.25) (layer F.Cu) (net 4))
 (segment (start 153.45 91.6) (end 154.1 91.6) (width 0.25) (layer F.Cu) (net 4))
 (segment (start 152.595 93.905) (end 153.3 93.2) (width 0.25) (layer F.Cu) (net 2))
 (segment (start 151.075 93.905) (end 152.595 93.905) (width 0.25) (layer F.Cu) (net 2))
 (segment (start 153.3 93.2) (end 154.1 93.2) (width 0.25) (layer F.Cu) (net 2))
 (segment (start 156.9 91.6) (end 157.5 91) (width 0.25) (layer F.Cu) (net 8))
 (segment (start 157.5 91) (end 158.9 91) (width 0.25) (layer F.Cu) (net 8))
 (segment (start 155.9 91.6) (end 156.9 91.6) (width 0.25) (layer F.Cu) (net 8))
 (segment (start 155.9 90.8) (end 155.9 90.3) (width 0.25) (layer F.Cu) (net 7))
 (segment (start 157.2 89) (end 158.05 89) (width 0.25) (layer F.Cu) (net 7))
 (segment (start 155.9 90.3) (end 157.2 89) (width 0.25) (layer F.Cu) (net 7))
 (segment (start 158.05 89) (end 158.9 89) (width 0.25) (layer F.Cu) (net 7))
 (segment (start 156.9 92.4) (end 157.5 93) (width 0.25) (layer F.Cu) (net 9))
 (segment (start 155.9 92.4) (end 156.9 92.4) (width 0.25) (layer F.Cu) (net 9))
 (segment (start 155.9 93.2) (end 155.9 93.7) (width 0.25) (layer F.Cu) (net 10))
 (segment (start 155.9 93.7) (end 157.2 95) (width 0.25) (layer F.Cu) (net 10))
 (segment (start 157.2 95) (end 158.05 95) (width 0.25) (layer F.Cu) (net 10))
 (segment (start 158.05 95) (end 158.9 95) (width 0.25) (layer F.Cu) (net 10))
 (via (at 155 96) (size 0.8) (drill 0.4) (layers F.Cu B.Cu) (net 6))
 (via (at 135.5 94) (size 0.8) (drill 0.4) (layers F.Cu B.Cu) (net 6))
 (via (at 135.5 88.5) (size 0.8) (drill 0.4) (layers F.Cu B.Cu) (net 6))
 (via (at 142.5 90.5) (size 0.8) (drill 0.4) (layers F.Cu B.Cu) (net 1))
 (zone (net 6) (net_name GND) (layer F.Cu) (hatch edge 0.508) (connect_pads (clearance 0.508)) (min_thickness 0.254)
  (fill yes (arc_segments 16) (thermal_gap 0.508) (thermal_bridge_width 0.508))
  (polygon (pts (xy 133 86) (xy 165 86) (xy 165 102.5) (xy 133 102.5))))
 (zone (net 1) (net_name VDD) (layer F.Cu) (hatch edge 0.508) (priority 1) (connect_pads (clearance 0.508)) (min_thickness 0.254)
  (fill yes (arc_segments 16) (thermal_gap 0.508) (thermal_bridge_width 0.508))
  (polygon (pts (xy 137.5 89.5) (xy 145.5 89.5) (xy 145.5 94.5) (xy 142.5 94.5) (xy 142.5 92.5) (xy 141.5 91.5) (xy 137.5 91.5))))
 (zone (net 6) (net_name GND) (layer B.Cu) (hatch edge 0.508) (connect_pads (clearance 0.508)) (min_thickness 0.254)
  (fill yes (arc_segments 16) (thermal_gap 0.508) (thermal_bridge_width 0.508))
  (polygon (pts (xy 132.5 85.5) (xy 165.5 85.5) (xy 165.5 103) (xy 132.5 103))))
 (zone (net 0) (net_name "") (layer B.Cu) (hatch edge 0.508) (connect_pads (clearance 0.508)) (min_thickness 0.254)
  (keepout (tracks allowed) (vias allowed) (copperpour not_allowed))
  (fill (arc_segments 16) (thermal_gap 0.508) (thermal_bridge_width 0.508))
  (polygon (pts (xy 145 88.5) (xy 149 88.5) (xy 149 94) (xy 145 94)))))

